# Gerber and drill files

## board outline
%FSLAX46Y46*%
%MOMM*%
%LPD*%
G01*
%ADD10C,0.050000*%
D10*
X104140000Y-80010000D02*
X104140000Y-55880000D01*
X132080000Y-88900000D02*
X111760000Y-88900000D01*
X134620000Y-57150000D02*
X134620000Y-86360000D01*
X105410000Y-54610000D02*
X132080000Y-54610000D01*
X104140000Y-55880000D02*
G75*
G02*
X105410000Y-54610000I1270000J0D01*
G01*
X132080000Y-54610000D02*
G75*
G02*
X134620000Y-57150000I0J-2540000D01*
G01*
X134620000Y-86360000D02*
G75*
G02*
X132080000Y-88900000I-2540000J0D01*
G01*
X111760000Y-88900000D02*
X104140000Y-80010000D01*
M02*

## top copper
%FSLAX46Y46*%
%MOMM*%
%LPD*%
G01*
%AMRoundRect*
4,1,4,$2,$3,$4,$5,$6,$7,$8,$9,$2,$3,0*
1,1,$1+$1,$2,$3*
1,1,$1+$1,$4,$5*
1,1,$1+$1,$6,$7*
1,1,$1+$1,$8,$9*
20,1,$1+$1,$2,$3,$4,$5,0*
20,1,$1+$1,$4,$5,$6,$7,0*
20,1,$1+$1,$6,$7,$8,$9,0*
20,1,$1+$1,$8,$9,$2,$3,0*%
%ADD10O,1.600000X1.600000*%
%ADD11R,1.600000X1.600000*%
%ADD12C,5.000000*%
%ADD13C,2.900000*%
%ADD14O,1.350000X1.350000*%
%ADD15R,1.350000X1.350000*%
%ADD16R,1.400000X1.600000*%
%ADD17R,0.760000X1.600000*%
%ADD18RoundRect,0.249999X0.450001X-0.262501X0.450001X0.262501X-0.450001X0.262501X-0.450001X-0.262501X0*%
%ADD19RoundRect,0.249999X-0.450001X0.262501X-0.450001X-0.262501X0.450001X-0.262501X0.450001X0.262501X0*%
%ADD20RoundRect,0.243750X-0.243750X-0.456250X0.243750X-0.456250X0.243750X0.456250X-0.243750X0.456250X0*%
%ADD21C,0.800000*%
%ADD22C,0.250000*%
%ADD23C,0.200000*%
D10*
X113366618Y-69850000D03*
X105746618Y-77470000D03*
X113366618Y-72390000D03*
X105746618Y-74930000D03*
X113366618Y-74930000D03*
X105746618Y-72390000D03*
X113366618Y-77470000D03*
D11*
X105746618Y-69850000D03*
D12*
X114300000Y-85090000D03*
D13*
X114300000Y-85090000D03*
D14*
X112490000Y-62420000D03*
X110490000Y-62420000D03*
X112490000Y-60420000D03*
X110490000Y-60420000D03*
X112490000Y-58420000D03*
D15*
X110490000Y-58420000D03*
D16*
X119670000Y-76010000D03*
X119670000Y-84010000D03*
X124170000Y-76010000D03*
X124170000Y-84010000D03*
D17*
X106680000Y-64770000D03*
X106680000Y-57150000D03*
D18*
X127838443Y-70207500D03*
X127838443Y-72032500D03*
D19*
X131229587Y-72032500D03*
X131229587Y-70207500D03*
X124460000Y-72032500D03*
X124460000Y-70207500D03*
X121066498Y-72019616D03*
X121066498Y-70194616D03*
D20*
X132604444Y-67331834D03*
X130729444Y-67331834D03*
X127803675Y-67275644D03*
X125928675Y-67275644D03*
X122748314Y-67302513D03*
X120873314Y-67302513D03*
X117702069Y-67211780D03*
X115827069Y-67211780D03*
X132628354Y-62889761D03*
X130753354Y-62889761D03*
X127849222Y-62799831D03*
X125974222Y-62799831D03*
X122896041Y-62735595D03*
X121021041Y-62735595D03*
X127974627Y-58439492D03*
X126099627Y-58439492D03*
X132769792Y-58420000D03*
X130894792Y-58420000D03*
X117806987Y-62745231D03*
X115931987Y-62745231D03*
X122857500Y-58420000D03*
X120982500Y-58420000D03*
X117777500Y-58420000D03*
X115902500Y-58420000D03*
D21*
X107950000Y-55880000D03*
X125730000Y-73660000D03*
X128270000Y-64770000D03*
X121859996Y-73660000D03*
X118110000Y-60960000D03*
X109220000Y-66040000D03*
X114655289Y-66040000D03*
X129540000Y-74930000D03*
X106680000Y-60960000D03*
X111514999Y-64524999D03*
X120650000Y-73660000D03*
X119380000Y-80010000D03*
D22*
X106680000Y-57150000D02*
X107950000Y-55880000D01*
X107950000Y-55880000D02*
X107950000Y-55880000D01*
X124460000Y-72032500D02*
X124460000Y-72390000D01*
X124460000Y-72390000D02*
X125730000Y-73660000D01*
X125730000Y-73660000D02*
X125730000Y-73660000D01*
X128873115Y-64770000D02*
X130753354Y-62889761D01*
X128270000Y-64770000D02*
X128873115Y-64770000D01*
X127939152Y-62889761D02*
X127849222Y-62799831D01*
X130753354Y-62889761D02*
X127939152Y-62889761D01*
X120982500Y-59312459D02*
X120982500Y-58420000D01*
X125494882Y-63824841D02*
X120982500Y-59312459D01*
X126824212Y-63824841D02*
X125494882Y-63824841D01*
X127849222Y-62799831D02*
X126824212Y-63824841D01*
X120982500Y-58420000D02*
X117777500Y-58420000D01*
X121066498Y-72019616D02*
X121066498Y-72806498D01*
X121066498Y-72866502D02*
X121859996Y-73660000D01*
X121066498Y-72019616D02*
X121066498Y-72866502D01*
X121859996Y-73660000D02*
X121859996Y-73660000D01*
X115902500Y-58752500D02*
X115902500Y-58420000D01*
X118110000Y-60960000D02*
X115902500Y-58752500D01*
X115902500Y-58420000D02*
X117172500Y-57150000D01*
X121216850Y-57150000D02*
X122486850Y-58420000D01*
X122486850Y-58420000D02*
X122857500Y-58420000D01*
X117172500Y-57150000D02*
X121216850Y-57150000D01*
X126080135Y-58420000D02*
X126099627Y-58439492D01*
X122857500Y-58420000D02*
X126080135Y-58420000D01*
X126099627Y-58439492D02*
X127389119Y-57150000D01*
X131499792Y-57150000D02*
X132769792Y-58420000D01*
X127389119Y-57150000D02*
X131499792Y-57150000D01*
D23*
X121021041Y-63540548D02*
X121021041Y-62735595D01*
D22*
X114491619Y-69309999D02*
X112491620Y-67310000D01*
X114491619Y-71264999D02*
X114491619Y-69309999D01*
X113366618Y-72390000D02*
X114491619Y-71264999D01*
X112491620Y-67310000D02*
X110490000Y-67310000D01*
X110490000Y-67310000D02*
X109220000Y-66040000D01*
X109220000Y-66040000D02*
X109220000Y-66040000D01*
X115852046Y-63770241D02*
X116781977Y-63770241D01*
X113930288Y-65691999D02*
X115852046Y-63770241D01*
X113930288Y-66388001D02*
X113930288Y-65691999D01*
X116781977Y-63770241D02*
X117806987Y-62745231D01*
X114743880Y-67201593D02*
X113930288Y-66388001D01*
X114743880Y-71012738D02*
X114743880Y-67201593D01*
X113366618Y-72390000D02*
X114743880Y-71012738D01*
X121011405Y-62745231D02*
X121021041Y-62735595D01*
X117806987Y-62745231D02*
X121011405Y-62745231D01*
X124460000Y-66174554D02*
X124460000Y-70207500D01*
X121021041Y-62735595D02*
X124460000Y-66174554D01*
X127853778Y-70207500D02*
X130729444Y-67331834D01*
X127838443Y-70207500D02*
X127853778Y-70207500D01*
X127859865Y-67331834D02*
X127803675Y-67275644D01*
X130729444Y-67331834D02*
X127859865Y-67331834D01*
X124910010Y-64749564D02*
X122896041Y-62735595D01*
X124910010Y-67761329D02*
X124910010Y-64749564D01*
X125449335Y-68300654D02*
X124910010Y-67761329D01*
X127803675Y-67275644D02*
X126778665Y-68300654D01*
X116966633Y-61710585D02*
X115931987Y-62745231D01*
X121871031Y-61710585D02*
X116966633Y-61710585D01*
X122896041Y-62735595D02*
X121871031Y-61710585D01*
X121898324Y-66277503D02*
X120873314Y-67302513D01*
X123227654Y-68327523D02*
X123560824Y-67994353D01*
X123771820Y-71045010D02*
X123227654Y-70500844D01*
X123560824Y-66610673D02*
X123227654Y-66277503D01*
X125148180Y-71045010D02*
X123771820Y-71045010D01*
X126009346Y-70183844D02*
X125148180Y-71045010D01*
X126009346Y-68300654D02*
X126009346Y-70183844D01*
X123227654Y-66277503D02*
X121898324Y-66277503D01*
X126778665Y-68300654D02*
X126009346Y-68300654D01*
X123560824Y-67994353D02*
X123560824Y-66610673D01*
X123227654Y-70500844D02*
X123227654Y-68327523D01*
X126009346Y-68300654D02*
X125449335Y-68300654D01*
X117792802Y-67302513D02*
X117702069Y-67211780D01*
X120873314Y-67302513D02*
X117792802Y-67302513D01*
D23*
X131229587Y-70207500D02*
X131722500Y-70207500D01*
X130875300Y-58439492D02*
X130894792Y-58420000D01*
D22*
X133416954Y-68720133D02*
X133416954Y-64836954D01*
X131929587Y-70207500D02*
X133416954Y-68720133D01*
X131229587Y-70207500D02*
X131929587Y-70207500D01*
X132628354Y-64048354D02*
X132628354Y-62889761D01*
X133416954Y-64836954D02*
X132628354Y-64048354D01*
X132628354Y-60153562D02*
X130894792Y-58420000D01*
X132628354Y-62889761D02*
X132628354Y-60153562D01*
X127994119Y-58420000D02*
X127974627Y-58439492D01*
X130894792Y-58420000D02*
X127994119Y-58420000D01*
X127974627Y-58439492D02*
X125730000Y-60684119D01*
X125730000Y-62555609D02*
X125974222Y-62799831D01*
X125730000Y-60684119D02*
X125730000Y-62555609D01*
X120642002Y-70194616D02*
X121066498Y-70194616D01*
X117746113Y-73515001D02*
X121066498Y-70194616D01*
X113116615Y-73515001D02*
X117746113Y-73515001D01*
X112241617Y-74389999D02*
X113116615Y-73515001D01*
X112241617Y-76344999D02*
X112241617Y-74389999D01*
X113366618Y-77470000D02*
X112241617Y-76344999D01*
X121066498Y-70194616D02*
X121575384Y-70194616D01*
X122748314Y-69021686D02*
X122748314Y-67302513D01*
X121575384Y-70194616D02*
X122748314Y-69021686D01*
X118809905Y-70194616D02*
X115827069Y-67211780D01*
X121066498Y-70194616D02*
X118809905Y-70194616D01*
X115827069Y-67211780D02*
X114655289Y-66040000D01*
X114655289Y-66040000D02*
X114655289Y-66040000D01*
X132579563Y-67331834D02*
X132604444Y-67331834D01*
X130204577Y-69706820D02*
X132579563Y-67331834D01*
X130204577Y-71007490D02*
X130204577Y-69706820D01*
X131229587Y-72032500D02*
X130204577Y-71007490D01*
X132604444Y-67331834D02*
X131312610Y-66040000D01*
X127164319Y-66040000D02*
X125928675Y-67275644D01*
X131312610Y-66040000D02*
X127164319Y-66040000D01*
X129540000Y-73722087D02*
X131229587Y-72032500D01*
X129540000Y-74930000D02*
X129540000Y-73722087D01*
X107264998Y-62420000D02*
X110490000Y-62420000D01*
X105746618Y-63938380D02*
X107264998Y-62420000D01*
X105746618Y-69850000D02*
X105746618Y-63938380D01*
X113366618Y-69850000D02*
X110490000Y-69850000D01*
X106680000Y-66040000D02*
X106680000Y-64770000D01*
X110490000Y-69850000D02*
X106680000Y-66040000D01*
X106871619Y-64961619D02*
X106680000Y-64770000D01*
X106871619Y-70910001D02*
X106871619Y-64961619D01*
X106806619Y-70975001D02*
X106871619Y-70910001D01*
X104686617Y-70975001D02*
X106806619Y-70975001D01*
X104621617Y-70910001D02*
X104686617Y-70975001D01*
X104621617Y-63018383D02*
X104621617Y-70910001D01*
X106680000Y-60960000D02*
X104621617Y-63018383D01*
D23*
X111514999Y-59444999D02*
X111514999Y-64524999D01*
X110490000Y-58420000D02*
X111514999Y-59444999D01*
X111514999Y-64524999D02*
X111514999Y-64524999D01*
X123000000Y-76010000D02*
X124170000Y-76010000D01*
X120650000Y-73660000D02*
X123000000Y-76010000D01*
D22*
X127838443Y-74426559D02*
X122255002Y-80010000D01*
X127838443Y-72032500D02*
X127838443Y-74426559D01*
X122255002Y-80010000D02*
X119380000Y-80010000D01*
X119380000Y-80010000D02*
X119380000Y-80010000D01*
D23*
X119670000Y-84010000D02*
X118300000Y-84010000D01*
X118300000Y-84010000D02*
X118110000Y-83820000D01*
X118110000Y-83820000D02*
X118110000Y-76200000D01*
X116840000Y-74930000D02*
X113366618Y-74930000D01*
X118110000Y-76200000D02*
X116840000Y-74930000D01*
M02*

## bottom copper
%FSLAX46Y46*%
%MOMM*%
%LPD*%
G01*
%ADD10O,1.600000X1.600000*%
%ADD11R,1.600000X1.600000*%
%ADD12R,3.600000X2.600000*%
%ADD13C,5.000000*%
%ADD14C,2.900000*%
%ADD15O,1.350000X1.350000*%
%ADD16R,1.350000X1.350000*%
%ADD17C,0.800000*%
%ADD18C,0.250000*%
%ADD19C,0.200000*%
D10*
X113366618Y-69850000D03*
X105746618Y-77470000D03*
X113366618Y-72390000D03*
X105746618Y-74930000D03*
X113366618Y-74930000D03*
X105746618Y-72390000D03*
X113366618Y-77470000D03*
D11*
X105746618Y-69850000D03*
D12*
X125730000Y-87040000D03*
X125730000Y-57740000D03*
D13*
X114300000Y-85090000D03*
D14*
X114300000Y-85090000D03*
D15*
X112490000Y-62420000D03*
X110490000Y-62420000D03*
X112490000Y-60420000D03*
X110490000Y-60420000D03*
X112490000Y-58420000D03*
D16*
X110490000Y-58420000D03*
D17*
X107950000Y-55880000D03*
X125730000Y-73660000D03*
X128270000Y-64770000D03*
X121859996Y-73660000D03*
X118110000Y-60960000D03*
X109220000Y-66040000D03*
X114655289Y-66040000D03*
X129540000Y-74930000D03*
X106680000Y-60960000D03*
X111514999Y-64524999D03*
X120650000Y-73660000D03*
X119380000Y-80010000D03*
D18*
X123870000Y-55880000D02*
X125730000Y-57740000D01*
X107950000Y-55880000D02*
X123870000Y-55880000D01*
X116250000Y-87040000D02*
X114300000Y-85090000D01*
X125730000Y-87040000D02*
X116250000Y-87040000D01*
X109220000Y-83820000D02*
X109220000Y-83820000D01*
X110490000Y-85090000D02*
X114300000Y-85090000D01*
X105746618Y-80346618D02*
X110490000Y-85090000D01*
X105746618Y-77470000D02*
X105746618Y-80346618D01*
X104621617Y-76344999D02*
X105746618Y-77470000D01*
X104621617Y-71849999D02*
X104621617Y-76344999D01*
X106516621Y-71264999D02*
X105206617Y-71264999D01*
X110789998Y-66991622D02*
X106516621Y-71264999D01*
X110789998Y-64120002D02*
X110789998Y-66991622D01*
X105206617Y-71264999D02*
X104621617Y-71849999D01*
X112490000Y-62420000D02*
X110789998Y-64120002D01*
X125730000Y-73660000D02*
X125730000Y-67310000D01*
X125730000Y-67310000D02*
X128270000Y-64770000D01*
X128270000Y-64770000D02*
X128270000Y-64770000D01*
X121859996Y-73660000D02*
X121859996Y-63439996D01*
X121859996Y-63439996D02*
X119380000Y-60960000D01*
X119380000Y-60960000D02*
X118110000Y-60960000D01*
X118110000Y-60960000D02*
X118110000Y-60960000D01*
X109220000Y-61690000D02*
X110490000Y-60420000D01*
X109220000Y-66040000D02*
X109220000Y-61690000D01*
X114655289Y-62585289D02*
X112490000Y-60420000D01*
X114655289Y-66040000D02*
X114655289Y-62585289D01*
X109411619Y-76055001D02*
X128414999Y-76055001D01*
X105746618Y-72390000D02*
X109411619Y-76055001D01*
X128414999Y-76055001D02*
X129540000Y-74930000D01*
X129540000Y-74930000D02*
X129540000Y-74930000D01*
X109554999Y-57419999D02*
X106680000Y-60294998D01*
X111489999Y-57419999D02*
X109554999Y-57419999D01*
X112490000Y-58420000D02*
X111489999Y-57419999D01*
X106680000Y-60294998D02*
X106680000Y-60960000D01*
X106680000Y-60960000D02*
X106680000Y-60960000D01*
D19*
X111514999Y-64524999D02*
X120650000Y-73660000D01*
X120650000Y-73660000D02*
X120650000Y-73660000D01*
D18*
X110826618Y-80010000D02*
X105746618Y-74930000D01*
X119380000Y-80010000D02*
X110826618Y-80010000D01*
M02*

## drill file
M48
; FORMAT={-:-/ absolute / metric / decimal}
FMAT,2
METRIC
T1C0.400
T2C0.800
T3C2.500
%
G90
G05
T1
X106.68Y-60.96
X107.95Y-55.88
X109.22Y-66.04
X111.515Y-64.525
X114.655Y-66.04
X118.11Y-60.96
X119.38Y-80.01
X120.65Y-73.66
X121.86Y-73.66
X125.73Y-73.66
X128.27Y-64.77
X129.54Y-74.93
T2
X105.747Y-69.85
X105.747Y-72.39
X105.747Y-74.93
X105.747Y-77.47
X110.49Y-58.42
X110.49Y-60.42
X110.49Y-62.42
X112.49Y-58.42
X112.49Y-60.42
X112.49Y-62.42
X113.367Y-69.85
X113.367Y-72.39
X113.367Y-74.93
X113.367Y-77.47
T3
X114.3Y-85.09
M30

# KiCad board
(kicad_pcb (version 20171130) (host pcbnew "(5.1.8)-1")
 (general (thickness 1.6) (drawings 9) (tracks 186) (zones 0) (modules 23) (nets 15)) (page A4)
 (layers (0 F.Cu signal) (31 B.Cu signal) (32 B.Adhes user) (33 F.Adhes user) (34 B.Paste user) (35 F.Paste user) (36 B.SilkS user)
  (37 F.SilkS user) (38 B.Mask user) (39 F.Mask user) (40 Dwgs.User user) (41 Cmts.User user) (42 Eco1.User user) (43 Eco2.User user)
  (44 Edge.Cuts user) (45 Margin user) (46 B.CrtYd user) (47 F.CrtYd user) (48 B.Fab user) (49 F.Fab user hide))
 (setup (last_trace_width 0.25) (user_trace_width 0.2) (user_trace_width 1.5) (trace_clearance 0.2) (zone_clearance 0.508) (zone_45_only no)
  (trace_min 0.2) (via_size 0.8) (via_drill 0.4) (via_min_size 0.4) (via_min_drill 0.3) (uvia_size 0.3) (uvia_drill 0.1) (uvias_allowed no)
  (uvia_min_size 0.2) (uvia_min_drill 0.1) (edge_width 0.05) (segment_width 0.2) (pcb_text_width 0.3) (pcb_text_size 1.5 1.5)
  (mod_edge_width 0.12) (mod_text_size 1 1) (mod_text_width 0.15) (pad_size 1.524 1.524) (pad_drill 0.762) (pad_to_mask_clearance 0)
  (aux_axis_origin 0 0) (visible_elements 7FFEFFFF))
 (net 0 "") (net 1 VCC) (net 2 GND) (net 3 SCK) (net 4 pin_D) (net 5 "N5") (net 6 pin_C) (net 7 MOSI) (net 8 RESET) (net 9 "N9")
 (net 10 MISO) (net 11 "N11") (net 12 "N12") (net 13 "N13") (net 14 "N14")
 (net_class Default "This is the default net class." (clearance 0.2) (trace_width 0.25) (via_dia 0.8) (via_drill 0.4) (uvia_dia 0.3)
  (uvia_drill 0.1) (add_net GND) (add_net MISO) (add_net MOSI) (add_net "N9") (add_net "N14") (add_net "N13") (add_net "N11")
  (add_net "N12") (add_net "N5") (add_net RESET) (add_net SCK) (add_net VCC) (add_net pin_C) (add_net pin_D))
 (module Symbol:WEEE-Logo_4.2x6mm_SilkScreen (layer F.Cu) (at 129.54 81.28 90)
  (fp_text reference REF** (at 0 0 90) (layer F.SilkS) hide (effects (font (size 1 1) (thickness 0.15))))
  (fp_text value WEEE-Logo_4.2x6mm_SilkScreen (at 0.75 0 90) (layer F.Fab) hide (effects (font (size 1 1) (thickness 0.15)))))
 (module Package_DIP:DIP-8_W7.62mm (layer F.Cu) (at 105.746618 69.85)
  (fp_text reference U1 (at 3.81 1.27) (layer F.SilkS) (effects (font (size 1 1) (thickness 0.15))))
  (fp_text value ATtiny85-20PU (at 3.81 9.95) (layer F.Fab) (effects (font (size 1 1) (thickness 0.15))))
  (pad 8 thru_hole oval (at 7.62 0) (size 1.6 1.6) (drill 0.8) (layers *.Cu *.Mask) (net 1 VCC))
  (pad 4 thru_hole oval (at 0 7.62) (size 1.6 1.6) (drill 0.8) (layers *.Cu *.Mask) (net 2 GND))
  (pad 7 thru_hole oval (at 7.62 2.54) (size 1.6 1.6) (drill 0.8) (layers *.Cu *.Mask) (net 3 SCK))
  (pad 3 thru_hole oval (at 0 5.08) (size 1.6 1.6) (drill 0.8) (layers *.Cu *.Mask) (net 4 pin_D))
  (pad 6 thru_hole oval (at 7.62 5.08) (size 1.6 1.6) (drill 0.8) (layers *.Cu *.Mask) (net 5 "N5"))
  (pad 2 thru_hole oval (at 0 2.54) (size 1.6 1.6) (drill 0.8) (layers *.Cu *.Mask) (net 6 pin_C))
  (pad 5 thru_hole oval (at 7.62 7.62) (size 1.6 1.6) (drill 0.8) (layers *.Cu *.Mask) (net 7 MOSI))
  (pad 1 thru_hole rect (at 0 0) (size 1.6 1.6) (drill 0.8) (layers *.Cu *.Mask) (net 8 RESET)))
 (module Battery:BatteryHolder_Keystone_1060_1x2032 (layer B.Cu) (at 125.73 72.39 270)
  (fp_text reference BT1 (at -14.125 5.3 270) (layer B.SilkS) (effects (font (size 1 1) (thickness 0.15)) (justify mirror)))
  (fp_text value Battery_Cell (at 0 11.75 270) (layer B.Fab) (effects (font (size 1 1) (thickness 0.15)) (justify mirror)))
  (pad 2 smd rect (at 14.65 0 90) (size 2.6 3.6) (layers B.Cu B.Paste B.Mask) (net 2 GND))
  (pad 1 smd rect (at -14.65 0 90) (size 2.6 3.6) (layers B.Cu B.Paste B.Mask) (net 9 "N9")))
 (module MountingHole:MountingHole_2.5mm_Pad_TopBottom (layer F.Cu) (at 114.3 85.09)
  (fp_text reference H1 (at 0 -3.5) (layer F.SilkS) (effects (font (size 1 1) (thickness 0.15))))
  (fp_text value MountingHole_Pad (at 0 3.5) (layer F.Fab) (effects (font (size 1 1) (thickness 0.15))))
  (pad 1 connect circle (at 0 0) (size 5 5) (layers B.Cu B.Mask) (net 2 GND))
  (pad 1 connect circle (at 0 0) (size 5 5) (layers F.Cu F.Mask) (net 2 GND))
  (pad 1 thru_hole circle (at 0 0) (size 2.9 2.9) (drill 2.5) (layers *.Cu *.Mask) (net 2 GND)))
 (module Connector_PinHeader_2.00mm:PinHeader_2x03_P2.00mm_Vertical (layer F.Cu) (at 110.49 58.42)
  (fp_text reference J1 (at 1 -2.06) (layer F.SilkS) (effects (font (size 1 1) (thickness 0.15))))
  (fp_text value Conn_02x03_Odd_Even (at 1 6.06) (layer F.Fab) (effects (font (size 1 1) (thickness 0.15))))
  (pad 6 thru_hole oval (at 2 4) (size 1.35 1.35) (drill 0.8) (layers *.Cu *.Mask) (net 2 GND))
  (pad 5 thru_hole oval (at 0 4) (size 1.35 1.35) (drill 0.8) (layers *.Cu *.Mask) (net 8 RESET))
  (pad 4 thru_hole oval (at 2 2) (size 1.35 1.35) (drill 0.8) (layers *.Cu *.Mask) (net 7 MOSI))
  (pad 3 thru_hole oval (at 0 2) (size 1.35 1.35) (drill 0.8) (layers *.Cu *.Mask) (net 3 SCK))
  (pad 2 thru_hole oval (at 2 0) (size 1.35 1.35) (drill 0.8) (layers *.Cu *.Mask) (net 1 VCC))
  (pad 1 thru_hole rect (at 0 0) (size 1.35 1.35) (drill 0.8) (layers *.Cu *.Mask) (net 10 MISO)))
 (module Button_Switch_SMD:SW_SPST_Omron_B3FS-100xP (layer F.Cu) (at 121.92 80.01 90)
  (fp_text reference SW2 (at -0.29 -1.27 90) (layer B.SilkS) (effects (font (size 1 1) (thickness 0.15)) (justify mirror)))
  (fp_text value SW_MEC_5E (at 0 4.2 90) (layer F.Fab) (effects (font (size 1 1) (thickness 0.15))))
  (pad 2 smd rect (at 4 -2.25 270) (size 1.6 1.4) (layers F.Cu F.Paste F.Mask))
  (pad 1 smd rect (at -4 -2.25 270) (size 1.6 1.4) (layers F.Cu F.Paste F.Mask) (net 5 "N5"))
  (pad 4 smd rect (at 4 2.25 270) (size 1.6 1.4) (layers F.Cu F.Paste F.Mask) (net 10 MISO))
  (pad 3 smd rect (at -4 2.25 270) (size 1.6 1.4) (layers F.Cu F.Paste F.Mask)))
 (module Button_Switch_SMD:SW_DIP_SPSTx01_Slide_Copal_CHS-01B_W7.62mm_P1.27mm (layer F.Cu) (at 106.68 60.96 90)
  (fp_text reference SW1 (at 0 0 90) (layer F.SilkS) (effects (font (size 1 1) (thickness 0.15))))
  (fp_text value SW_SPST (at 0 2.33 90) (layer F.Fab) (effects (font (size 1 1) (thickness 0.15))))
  (pad 1 smd rect (at -3.81 0 90) (size 1.6 0.76) (layers F.Cu F.Paste F.Mask) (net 1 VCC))
  (pad 2 smd rect (at 3.81 0 90) (size 1.6 0.76) (layers F.Cu F.Paste F.Mask) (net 9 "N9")))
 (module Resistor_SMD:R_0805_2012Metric (layer F.Cu) (at 127.838443 71.12 90)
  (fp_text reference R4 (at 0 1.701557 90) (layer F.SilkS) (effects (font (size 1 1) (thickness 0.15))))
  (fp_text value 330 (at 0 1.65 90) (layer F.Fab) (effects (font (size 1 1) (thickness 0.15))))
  (pad 2 smd roundrect (at 0.9125 0 90) (size 1.025 1.4) (layers F.Cu F.Paste F.Mask) (roundrect_rratio 0.2439014634146341) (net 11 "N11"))
  (pad 1 smd roundrect (at -0.9125 0 90) (size 1.025 1.4) (layers F.Cu F.Paste F.Mask) (roundrect_rratio 0.2439014634146341) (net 4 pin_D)))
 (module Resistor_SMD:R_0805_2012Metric (layer F.Cu) (at 131.229587 71.12 270)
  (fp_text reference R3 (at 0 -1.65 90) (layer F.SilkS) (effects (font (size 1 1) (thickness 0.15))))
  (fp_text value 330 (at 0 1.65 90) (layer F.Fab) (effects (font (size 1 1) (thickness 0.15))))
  (pad 2 smd roundrect (at 0.9125 0 270) (size 1.025 1.4) (layers F.Cu F.Paste F.Mask) (roundrect_rratio 0.2439014634146341) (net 6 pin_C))
  (pad 1 smd roundrect (at -0.9125 0 270) (size 1.025 1.4) (layers F.Cu F.Paste F.Mask) (roundrect_rratio 0.2439014634146341) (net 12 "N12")))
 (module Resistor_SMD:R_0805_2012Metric (layer F.Cu) (at 124.46 71.12 270)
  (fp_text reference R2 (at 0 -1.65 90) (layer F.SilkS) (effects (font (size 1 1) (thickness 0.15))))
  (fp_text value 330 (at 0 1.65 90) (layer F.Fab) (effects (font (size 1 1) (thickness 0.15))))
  (pad 2 smd roundrect (at 0.9125 0 270) (size 1.025 1.4) (layers F.Cu F.Paste F.Mask) (roundrect_rratio 0.2439014634146341) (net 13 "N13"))
  (pad 1 smd roundrect (at -0.9125 0 270) (size 1.025 1.4) (layers F.Cu F.Paste F.Mask) (roundrect_rratio 0.2439014634146341) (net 3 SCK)))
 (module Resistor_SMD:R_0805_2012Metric (layer F.Cu) (at 121.066498 71.107116 270)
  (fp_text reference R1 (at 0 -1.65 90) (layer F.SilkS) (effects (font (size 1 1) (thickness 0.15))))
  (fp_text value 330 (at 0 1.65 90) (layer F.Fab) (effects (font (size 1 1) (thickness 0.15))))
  (pad 2 smd roundrect (at 0.9125 0 270) (size 1.025 1.4) (layers F.Cu F.Paste F.Mask) (roundrect_rratio 0.2439014634146341) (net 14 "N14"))
  (pad 1 smd roundrect (at -0.9125 0 270) (size 1.025 1.4) (layers F.Cu F.Paste F.Mask) (roundrect_rratio 0.2439014634146341) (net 7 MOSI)))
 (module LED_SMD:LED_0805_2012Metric (layer F.Cu) (at 131.666944 67.331834)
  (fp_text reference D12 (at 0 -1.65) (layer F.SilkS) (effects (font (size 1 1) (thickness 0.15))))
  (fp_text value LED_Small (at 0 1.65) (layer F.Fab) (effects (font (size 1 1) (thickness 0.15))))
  (pad 2 smd roundrect (at 0.9375 0) (size 0.975 1.4) (layers F.Cu F.Paste F.Mask) (roundrect_rratio 0.25) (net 6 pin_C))
  (pad 1 smd roundrect (at -0.9375 0) (size 0.975 1.4) (layers F.Cu F.Paste F.Mask) (roundrect_rratio 0.25) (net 11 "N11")))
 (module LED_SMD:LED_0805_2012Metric (layer F.Cu) (at 126.866175 67.275644)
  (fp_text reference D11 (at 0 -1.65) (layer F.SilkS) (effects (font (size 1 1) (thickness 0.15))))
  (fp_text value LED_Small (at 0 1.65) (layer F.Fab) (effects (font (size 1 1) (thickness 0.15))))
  (pad 2 smd roundrect (at 0.9375 0) (size 0.975 1.4) (layers F.Cu F.Paste F.Mask) (roundrect_rratio 0.25) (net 11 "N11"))
  (pad 1 smd roundrect (at -0.9375 0) (size 0.975 1.4) (layers F.Cu F.Paste F.Mask) (roundrect_rratio 0.25) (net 6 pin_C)))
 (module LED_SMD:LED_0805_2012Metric (layer F.Cu) (at 121.810814 67.302513)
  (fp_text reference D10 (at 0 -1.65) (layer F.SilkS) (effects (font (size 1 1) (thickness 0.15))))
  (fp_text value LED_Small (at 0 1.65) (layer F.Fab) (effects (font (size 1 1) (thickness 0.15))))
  (pad 2 smd roundrect (at 0.9375 0) (size 0.975 1.4) (layers F.Cu F.Paste F.Mask) (roundrect_rratio 0.25) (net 7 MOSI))
  (pad 1 smd roundrect (at -0.9375 0) (size 0.975 1.4) (layers F.Cu F.Paste F.Mask) (roundrect_rratio 0.25) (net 11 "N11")))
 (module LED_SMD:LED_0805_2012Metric (layer F.Cu) (at 116.764569 67.21178)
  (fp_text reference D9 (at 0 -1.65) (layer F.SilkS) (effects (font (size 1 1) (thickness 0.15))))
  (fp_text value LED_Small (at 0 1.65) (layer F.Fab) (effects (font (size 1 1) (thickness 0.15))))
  (pad 2 smd roundrect (at 0.9375 0) (size 0.975 1.4) (layers F.Cu F.Paste F.Mask) (roundrect_rratio 0.25) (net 11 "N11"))
  (pad 1 smd roundrect (at -0.9375 0) (size 0.975 1.4) (layers F.Cu F.Paste F.Mask) (roundrect_rratio 0.25) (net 7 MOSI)))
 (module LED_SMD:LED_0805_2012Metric (layer F.Cu) (at 131.690854 62.889761)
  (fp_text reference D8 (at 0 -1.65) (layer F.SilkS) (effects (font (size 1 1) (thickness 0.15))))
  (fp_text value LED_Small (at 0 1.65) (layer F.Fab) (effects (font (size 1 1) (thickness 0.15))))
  (pad 2 smd roundrect (at 0.9375 0) (size 0.975 1.4) (layers F.Cu F.Paste F.Mask) (roundrect_rratio 0.25) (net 12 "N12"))
  (pad 1 smd roundrect (at -0.9375 0) (size 0.975 1.4) (layers F.Cu F.Paste F.Mask) (roundrect_rratio 0.25) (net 13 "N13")))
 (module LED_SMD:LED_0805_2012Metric (layer F.Cu) (at 126.911722 62.799831)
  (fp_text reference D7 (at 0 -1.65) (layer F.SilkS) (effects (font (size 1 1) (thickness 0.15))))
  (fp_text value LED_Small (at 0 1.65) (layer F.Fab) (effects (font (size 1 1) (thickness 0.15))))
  (pad 2 smd roundrect (at 0.9375 0) (size 0.975 1.4) (layers F.Cu F.Paste F.Mask) (roundrect_rratio 0.25) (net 13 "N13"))
  (pad 1 smd roundrect (at -0.9375 0) (size 0.975 1.4) (layers F.Cu F.Paste F.Mask) (roundrect_rratio 0.25) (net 12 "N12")))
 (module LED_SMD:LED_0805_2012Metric (layer F.Cu) (at 121.958541 62.735595)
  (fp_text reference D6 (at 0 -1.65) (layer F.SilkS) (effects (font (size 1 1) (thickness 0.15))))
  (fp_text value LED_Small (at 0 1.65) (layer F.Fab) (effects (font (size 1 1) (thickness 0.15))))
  (pad 2 smd roundrect (at 0.9375 0) (size 0.975 1.4) (layers F.Cu F.Paste F.Mask) (roundrect_rratio 0.25) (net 11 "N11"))
  (pad 1 smd roundrect (at -0.9375 0) (size 0.975 1.4) (layers F.Cu F.Paste F.Mask) (roundrect_rratio 0.25) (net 3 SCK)))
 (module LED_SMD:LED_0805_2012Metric (layer F.Cu) (at 127.037127 58.439492)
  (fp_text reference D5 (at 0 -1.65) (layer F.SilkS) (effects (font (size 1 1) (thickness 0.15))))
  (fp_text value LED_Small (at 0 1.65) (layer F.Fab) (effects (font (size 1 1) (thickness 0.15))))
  (pad 2 smd roundrect (at 0.9375 0) (size 0.975 1.4) (layers F.Cu F.Paste F.Mask) (roundrect_rratio 0.25) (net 12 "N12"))
  (pad 1 smd roundrect (at -0.9375 0) (size 0.975 1.4) (layers F.Cu F.Paste F.Mask) (roundrect_rratio 0.25) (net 14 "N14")))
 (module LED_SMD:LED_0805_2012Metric (layer F.Cu) (at 131.832292 58.42)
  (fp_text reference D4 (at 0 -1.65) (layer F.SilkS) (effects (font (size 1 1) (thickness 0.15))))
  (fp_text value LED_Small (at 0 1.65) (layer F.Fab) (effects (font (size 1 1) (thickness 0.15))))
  (pad 2 smd roundrect (at 0.9375 0) (size 0.975 1.4) (layers F.Cu F.Paste F.Mask) (roundrect_rratio 0.25) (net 14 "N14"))
  (pad 1 smd roundrect (at -0.9375 0) (size 0.975 1.4) (layers F.Cu F.Paste F.Mask) (roundrect_rratio 0.25) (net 12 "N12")))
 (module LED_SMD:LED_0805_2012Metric (layer F.Cu) (at 116.869487 62.745231)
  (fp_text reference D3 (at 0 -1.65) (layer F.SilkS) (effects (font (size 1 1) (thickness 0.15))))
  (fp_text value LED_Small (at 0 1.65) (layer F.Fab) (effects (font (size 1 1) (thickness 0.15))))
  (pad 2 smd roundrect (at 0.9375 0) (size 0.975 1.4) (layers F.Cu F.Paste F.Mask) (roundrect_rratio 0.25) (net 3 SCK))
  (pad 1 smd roundrect (at -0.9375 0) (size 0.975 1.4) (layers F.Cu F.Paste F.Mask) (roundrect_rratio 0.25) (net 11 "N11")))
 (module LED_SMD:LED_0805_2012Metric (layer F.Cu) (at 121.92 58.42)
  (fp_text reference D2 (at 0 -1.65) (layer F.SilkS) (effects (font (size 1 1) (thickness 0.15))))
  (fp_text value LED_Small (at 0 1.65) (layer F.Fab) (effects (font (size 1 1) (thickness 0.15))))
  (pad 2 smd roundrect (at 0.9375 0) (size 0.975 1.4) (layers F.Cu F.Paste F.Mask) (roundrect_rratio 0.25) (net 14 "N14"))
  (pad 1 smd roundrect (at -0.9375 0) (size 0.975 1.4) (layers F.Cu F.Paste F.Mask) (roundrect_rratio 0.25) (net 13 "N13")))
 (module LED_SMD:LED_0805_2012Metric (layer F.Cu) (at 116.84 58.42)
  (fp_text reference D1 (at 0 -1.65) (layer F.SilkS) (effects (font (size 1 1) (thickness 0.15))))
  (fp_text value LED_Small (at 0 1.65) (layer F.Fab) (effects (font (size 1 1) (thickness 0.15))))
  (pad 2 smd roundrect (at 0.9375 0) (size 0.975 1.4) (layers F.Cu F.Paste F.Mask) (roundrect_rratio 0.25) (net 13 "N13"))
  (pad 1 smd roundrect (at -0.9375 0) (size 0.975 1.4) (layers F.Cu F.Paste F.Mask) (roundrect_rratio 0.25) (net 14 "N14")))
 (gr_line (start 104.14 80.01) (end 104.14 55.88) (layer Edge.Cuts) (width 0.05))
 (gr_line (start 132.08 88.9) (end 111.76 88.9) (layer Edge.Cuts) (width 0.05))
 (gr_line (start 134.62 57.15) (end 134.62 86.36) (layer Edge.Cuts) (width 0.05))
 (gr_line (start 105.41 54.61) (end 132.08 54.61) (layer Edge.Cuts) (width 0.05))
 (gr_arc (start 105.41 55.88) (end 105.41 54.61) (angle -90) (layer Edge.Cuts) (width 0.05))
 (gr_arc (start 132.08 57.15) (end 134.62 57.15) (angle -90) (layer Edge.Cuts) (width 0.05))
 (gr_arc (start 132.08 86.36) (end 132.08 88.9) (angle -90) (layer Edge.Cuts) (width 0.05))
 (gr_line (start 111.76 88.9) (end 104.14 80.01) (layer Edge.Cuts) (width 0.05))
 (segment (start 106.68 57.15) (end 107.95 55.88) (width 0.25) (layer F.Cu) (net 9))
 (segment (start 107.95 55.88) (end 107.95 55.88) (width 0.25) (layer F.Cu) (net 9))
 (via (at 107.95 55.88) (size 0.8) (drill 0.4) (layers F.Cu B.Cu) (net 9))
 (segment (start 123.87 55.88) (end 125.73 57.74) (width 0.25) (layer B.Cu) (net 9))
 (segment (start 107.95 55.88) (end 123.87 55.88) (width 0.25) (layer B.Cu) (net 9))
 (segment (start 116.25 87.04) (end 114.3 85.09) (width 0.25) (layer B.Cu) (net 2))
 (segment (start 125.73 87.04) (end 116.25 87.04) (width 0.25) (layer B.Cu) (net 2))
 (segment (start 109.22 83.82) (end 109.22 83.82) (width 0.25) (layer B.Cu) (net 2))
 (segment (start 110.49 85.09) (end 114.3 85.09) (width 0.25) (layer B.Cu) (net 2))
 (segment (start 105.746618 80.346618) (end 110.49 85.09) (width 0.25) (layer B.Cu) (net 2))
 (segment (start 105.746618 77.47) (end 105.746618 80.346618) (width 0.25) (layer B.Cu) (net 2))
 (segment (start 104.621617 76.344999) (end 105.746618 77.47) (width 0.25) (layer B.Cu) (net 2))
 (segment (start 104.621617 71.849999) (end 104.621617 76.344999) (width 0.25) (layer B.Cu) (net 2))
 (segment (start 106.516621 71.264999) (end 105.206617 71.264999) (width 0.25) (layer B.Cu) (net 2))
 (segment (start 110.789998 66.991622) (end 106.516621 71.264999) (width 0.25) (layer B.Cu) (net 2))
 (segment (start 110.789998 64.120002) (end 110.789998 66.991622) (width 0.25) (layer B.Cu) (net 2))
 (segment (start 105.206617 71.264999) (end 104.621617 71.849999) (width 0.25) (layer B.Cu) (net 2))
 (segment (start 112.49 62.42) (end 110.789998 64.120002) (width 0.25) (layer B.Cu) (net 2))
 (segment (start 124.46 72.0325) (end 124.46 72.39) (width 0.25) (layer F.Cu) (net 13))
 (segment (start 124.46 72.39) (end 125.73 73.66) (width 0.25) (layer F.Cu) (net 13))
 (segment (start 125.73 73.66) (end 125.73 73.66) (width 0.25) (layer F.Cu) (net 13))
 (via (at 125.73 73.66) (size 0.8) (drill 0.4) (layers F.Cu B.Cu) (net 13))
 (segment (start 125.73 73.66) (end 125.73 67.31) (width 0.25) (layer B.Cu) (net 13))
 (segment (start 125.73 67.31) (end 128.27 64.77) (width 0.25) (layer B.Cu) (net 13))
 (segment (start 128.27 64.77) (end 128.27 64.77) (width 0.25) (layer B.Cu) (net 13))
 (via (at 128.27 64.77) (size 0.8) (drill 0.4) (layers F.Cu B.Cu) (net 13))
 (segment (start 128.873115 64.77) (end 130.753354 62.889761) (width 0.25) (layer F.Cu) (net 13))
 (segment (start 128.27 64.77) (end 128.873115 64.77) (width 0.25) (layer F.Cu) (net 13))
 (segment (start 127.939152 62.889761) (end 127.849222 62.799831) (width 0.25) (layer F.Cu) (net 13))
 (segment (start 130.753354 62.889761) (end 127.939152 62.889761) (width 0.25) (layer F.Cu) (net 13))
 (segment (start 120.9825 59.312459) (end 120.9825 58.42) (width 0.25) (layer F.Cu) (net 13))
 (segment (start 125.494882 63.824841) (end 120.9825 59.312459) (width 0.25) (layer F.Cu) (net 13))
 (segment (start 126.824212 63.824841) (end 125.494882 63.824841) (width 0.25) (layer F.Cu) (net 13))
 (segment (start 127.849222 62.799831) (end 126.824212 63.824841) (width 0.25) (layer F.Cu) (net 13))
 (segment (start 120.9825 58.42) (end 117.7775 58.42) (width 0.25) (layer F.Cu) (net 13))
 (segment (start 121.066498 72.019616) (end 121.066498 72.806498) (width 0.25) (layer F.Cu) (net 14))
 (segment (start 121.066498 72.866502) (end 121.859996 73.66) (width 0.25) (layer F.Cu) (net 14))
 (segment (start 121.066498 72.019616) (end 121.066498 72.866502) (width 0.25) (layer F.Cu) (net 14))
 (segment (start 121.859996 73.66) (end 121.859996 73.66) (width 0.25) (layer F.Cu) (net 14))
 (via (at 121.859996 73.66) (size 0.8) (drill 0.4) (layers F.Cu B.Cu) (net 14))
 (segment (start 121.859996 73.66) (end 121.859996 63.439996) (width 0.25) (layer B.Cu) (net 14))
 (segment (start 121.859996 63.439996) (end 119.38 60.96) (width 0.25) (layer B.Cu) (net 14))
 (segment (start 119.38 60.96) (end 118.11 60.96) (width 0.25) (layer B.Cu) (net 14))
 (segment (start 118.11 60.96) (end 118.11 60.96) (width 0.25) (layer B.Cu) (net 14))
 (via (at 118.11 60.96) (size 0.8) (drill 0.4) (layers F.Cu B.Cu) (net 14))
 (segment (start 115.9025 58.7525) (end 115.9025 58.42) (width 0.25) (layer F.Cu) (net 14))
 (segment (start 118.11 60.96) (end 115.9025 58.7525) (width 0.25) (layer F.Cu) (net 14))
 (segment (start 115.9025 58.42) (end 117.1725 57.15) (width 0.25) (layer F.Cu) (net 14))
 (segment (start 121.21685 57.15) (end 122.48685 58.42) (width 0.25) (layer F.Cu) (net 14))
 (segment (start 122.48685 58.42) (end 122.8575 58.42) (width 0.25) (layer F.Cu) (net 14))
 (segment (start 117.1725 57.15) (end 121.21685 57.15) (width 0.25) (layer F.Cu) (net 14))
 (segment (start 126.080135 58.42) (end 126.099627 58.439492) (width 0.25) (layer F.Cu) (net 14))
 (segment (start 122.8575 58.42) (end 126.080135 58.42) (width 0.25) (layer F.Cu) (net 14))
 (segment (start 126.099627 58.439492) (end 127.389119 57.15) (width 0.25) (layer F.Cu) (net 14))
 (segment (start 131.499792 57.15) (end 132.769792 58.42) (width 0.25) (layer F.Cu) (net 14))
 (segment (start 127.389119 57.15) (end 131.499792 57.15) (width 0.25) (layer F.Cu) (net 14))
 (segment (start 121.021041 63.540548) (end 121.021041 62.735595) (width 0.2) (layer F.Cu) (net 3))
 (segment (start 114.491619 69.309999) (end 112.49162 67.31) (width 0.25) (layer F.Cu) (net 3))
 (segment (start 114.491619 71.264999) (end 114.491619 69.309999) (width 0.25) (layer F.Cu) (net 3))
 (segment (start 113.366618 72.39) (end 114.491619 71.264999) (width 0.25) (layer F.Cu) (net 3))
 (segment (start 112.49162 67.31) (end 110.49 67.31) (width 0.25) (layer F.Cu) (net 3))
 (segment (start 110.49 67.31) (end 109.22 66.04) (width 0.25) (layer F.Cu) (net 3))
 (segment (start 109.22 66.04) (end 109.22 66.04) (width 0.25) (layer F.Cu) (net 3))
 (via (at 109.22 66.04) (size 0.8) (drill 0.4) (layers F.Cu B.Cu) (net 3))
 (segment (start 109.22 61.69) (end 110.49 60.42) (width 0.25) (layer B.Cu) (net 3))
 (segment (start 109.22 66.04) (end 109.22 61.69) (width 0.25) (layer B.Cu) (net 3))
 (segment (start 115.852046 63.770241) (end 116.781977 63.770241) (width 0.25) (layer F.Cu) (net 3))
 (segment (start 113.930288 65.691999) (end 115.852046 63.770241) (width 0.25) (layer F.Cu) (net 3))
 (segment (start 113.930288 66.388001) (end 113.930288 65.691999) (width 0.25) (layer F.Cu) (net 3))
 (segment (start 116.781977 63.770241) (end 117.806987 62.745231) (width 0.25) (layer F.Cu) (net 3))
 (segment (start 114.74388 67.201593) (end 113.930288 66.388001) (width 0.25) (layer F.Cu) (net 3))
 (segment (start 114.74388 71.012738) (end 114.74388 67.201593) (width 0.25) (layer F.Cu) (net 3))
 (segment (start 113.366618 72.39) (end 114.74388 71.012738) (width 0.25) (layer F.Cu) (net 3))
 (segment (start 121.011405 62.745231) (end 121.021041 62.735595) (width 0.25) (layer F.Cu) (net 3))
 (segment (start 117.806987 62.745231) (end 121.011405 62.745231) (width 0.25) (layer F.Cu) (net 3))
 (segment (start 124.46 66.174554) (end 124.46 70.2075) (width 0.25) (layer F.Cu) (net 3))
 (segment (start 121.021041 62.735595) (end 124.46 66.174554) (width 0.25) (layer F.Cu) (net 3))
 (segment (start 127.853778 70.2075) (end 130.729444 67.331834) (width 0.25) (layer F.Cu) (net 11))
 (segment (start 127.838443 70.2075) (end 127.853778 70.2075) (width 0.25) (layer F.Cu) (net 11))
 (segment (start 127.859865 67.331834) (end 127.803675 67.275644) (width 0.25) (layer F.Cu) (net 11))
 (segment (start 130.729444 67.331834) (end 127.859865 67.331834) (width 0.25) (layer F.Cu) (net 11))
 (segment (start 124.91001 64.749564) (end 122.896041 62.735595) (width 0.25) (layer F.Cu) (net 11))
 (segment (start 124.91001 67.761329) (end 124.91001 64.749564) (width 0.25) (layer F.Cu) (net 11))
 (segment (start 125.449335 68.300654) (end 124.91001 67.761329) (width 0.25) (layer F.Cu) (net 11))
 (segment (start 127.803675 67.275644) (end 126.778665 68.300654) (width 0.25) (layer F.Cu) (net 11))
 (segment (start 116.966633 61.710585) (end 115.931987 62.745231) (width 0.25) (layer F.Cu) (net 11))
 (segment (start 121.871031 61.710585) (end 116.966633 61.710585) (width 0.25) (layer F.Cu) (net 11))
 (segment (start 122.896041 62.735595) (end 121.871031 61.710585) (width 0.25) (layer F.Cu) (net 11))
 (segment (start 121.898324 66.277503) (end 120.873314 67.302513) (width 0.25) (layer F.Cu) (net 11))
 (segment (start 123.227654 68.327523) (end 123.560824 67.994353) (width 0.25) (layer F.Cu) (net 11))
 (segment (start 123.77182 71.04501) (end 123.227654 70.500844) (width 0.25) (layer F.Cu) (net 11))
 (segment (start 123.560824 66.610673) (end 123.227654 66.277503) (width 0.25) (layer F.Cu) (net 11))
 (segment (start 125.14818 71.04501) (end 123.77182 71.04501) (width 0.25) (layer F.Cu) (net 11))
 (segment (start 126.009346 70.183844) (end 125.14818 71.04501) (width 0.25) (layer F.Cu) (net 11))
 (segment (start 126.009346 68.300654) (end 126.009346 70.183844) (width 0.25) (layer F.Cu) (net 11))
 (segment (start 123.227654 66.277503) (end 121.898324 66.277503) (width 0.25) (layer F.Cu) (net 11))
 (segment (start 126.778665 68.300654) (end 126.009346 68.300654) (width 0.25) (layer F.Cu) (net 11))
 (segment (start 123.560824 67.994353) (end 123.560824 66.610673) (width 0.25) (layer F.Cu) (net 11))
 (segment (start 123.227654 70.500844) (end 123.227654 68.327523) (width 0.25) (layer F.Cu) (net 11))
 (segment (start 126.009346 68.300654) (end 125.449335 68.300654) (width 0.25) (layer F.Cu) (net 11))
 (segment (start 117.792802 67.302513) (end 117.702069 67.21178) (width 0.25) (layer F.Cu) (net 11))
 (segment (start 120.873314 67.302513) (end 117.792802 67.302513) (width 0.25) (layer F.Cu) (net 11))
 (segment (start 131.229587 70.2075) (end 131.7225 70.2075) (width 0.2) (layer F.Cu) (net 12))
 (segment (start 130.8753 58.439492) (end 130.894792 58.42) (width 0.2) (layer F.Cu) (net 12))
 (segment (start 133.416954 68.720133) (end 133.416954 64.836954) (width 0.25) (layer F.Cu) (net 12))
 (segment (start 131.929587 70.2075) (end 133.416954 68.720133) (width 0.25) (layer F.Cu) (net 12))
 (segment (start 131.229587 70.2075) (end 131.929587 70.2075) (width 0.25) (layer F.Cu) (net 12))
 (segment (start 132.628354 64.048354) (end 132.628354 62.889761) (width 0.25) (layer F.Cu) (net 12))
 (segment (start 133.416954 64.836954) (end 132.628354 64.048354) (width 0.25) (layer F.Cu) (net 12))
 (segment (start 132.628354 60.153562) (end 130.894792 58.42) (width 0.25) (layer F.Cu) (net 12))
 (segment (start 132.628354 62.889761) (end 132.628354 60.153562) (width 0.25) (layer F.Cu) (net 12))
 (segment (start 127.994119 58.42) (end 127.974627 58.439492) (width 0.25) (layer F.Cu) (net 12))
 (segment (start 130.894792 58.42) (end 127.994119 58.42) (width 0.25) (layer F.Cu) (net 12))
 (segment (start 127.974627 58.439492) (end 125.73 60.684119) (width 0.25) (layer F.Cu) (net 12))
 (segment (start 125.73 62.555609) (end 125.974222 62.799831) (width 0.25) (layer F.Cu) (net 12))
 (segment (start 125.73 60.684119) (end 125.73 62.555609) (width 0.25) (layer F.Cu) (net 12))
 (segment (start 120.642002 70.194616) (end 121.066498 70.194616) (width 0.25) (layer F.Cu) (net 7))
 (segment (start 117.746113 73.515001) (end 121.066498 70.194616) (width 0.25) (layer F.Cu) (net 7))
 (segment (start 113.116615 73.515001) (end 117.746113 73.515001) (width 0.25) (layer F.Cu) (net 7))
 (segment (start 112.241617 74.389999) (end 113.116615 73.515001) (width 0.25) (layer F.Cu) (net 7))
 (segment (start 112.241617 76.344999) (end 112.241617 74.389999) (width 0.25) (layer F.Cu) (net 7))
 (segment (start 113.366618 77.47) (end 112.241617 76.344999) (width 0.25) (layer F.Cu) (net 7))
 (segment (start 121.066498 70.194616) (end 121.575384 70.194616) (width 0.25) (layer F.Cu) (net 7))
 (segment (start 122.748314 69.021686) (end 122.748314 67.302513) (width 0.25) (layer F.Cu) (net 7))
 (segment (start 121.575384 70.194616) (end 122.748314 69.021686) (width 0.25) (layer F.Cu) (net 7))
 (segment (start 118.809905 70.194616) (end 115.827069 67.21178) (width 0.25) (layer F.Cu) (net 7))
 (segment (start 121.066498 70.194616) (end 118.809905 70.194616) (width 0.25) (layer F.Cu) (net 7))
 (segment (start 115.827069 67.21178) (end 114.655289 66.04) (width 0.25) (layer F.Cu) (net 7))
 (segment (start 114.655289 66.04) (end 114.655289 66.04) (width 0.25) (layer F.Cu) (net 7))
 (via (at 114.655289 66.04) (size 0.8) (drill 0.4) (layers F.Cu B.Cu) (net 7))
 (segment (start 114.655289 62.585289) (end 112.49 60.42) (width 0.25) (layer B.Cu) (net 7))
 (segment (start 114.655289 66.04) (end 114.655289 62.585289) (width 0.25) (layer B.Cu) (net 7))
 (segment (start 132.579563 67.331834) (end 132.604444 67.331834) (width 0.25) (layer F.Cu) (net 6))
 (segment (start 130.204577 69.70682) (end 132.579563 67.331834) (width 0.25) (layer F.Cu) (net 6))
 (segment (start 130.204577 71.00749) (end 130.204577 69.70682) (width 0.25) (layer F.Cu) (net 6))
 (segment (start 131.229587 72.0325) (end 130.204577 71.00749) (width 0.25) (layer F.Cu) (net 6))
 (segment (start 132.604444 67.331834) (end 131.31261 66.04) (width 0.25) (layer F.Cu) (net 6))
 (segment (start 127.164319 66.04) (end 125.928675 67.275644) (width 0.25) (layer F.Cu) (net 6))
 (segment (start 131.31261 66.04) (end 127.164319 66.04) (width 0.25) (layer F.Cu) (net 6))
 (segment (start 109.411619 76.055001) (end 128.414999 76.055001) (width 0.25) (layer B.Cu) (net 6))
 (segment (start 105.746618 72.39) (end 109.411619 76.055001) (width 0.25) (layer B.Cu) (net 6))
 (segment (start 128.414999 76.055001) (end 129.54 74.93) (width 0.25) (layer B.Cu) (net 6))
 (segment (start 129.54 74.93) (end 129.54 74.93) (width 0.25) (layer B.Cu) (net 6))
 (via (at 129.54 74.93) (size 0.8) (drill 0.4) (layers F.Cu B.Cu) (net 6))
 (segment (start 129.54 73.722087) (end 131.229587 72.0325) (width 0.25) (layer F.Cu) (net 6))
 (segment (start 129.54 74.93) (end 129.54 73.722087) (width 0.25) (layer F.Cu) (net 6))
 (segment (start 107.264998 62.42) (end 110.49 62.42) (width 0.25) (layer F.Cu) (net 8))
 (segment (start 105.746618 63.93838) (end 107.264998 62.42) (width 0.25) (layer F.Cu) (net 8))
 (segment (start 105.746618 69.85) (end 105.746618 63.93838) (width 0.25) (layer F.Cu) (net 8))
 (segment (start 113.366618 69.85) (end 110.49 69.85) (width 0.25) (layer F.Cu) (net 1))
 (segment (start 106.68 66.04) (end 106.68 64.77) (width 0.25) (layer F.Cu) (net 1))
 (segment (start 110.49 69.85) (end 106.68 66.04) (width 0.25) (layer F.Cu) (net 1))
 (segment (start 109.554999 57.419999) (end 106.68 60.294998) (width 0.25) (layer B.Cu) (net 1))
 (segment (start 111.489999 57.419999) (end 109.554999 57.419999) (width 0.25) (layer B.Cu) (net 1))
 (segment (start 112.49 58.42) (end 111.489999 57.419999) (width 0.25) (layer B.Cu) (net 1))
 (segment (start 106.68 60.294998) (end 106.68 60.96) (width 0.25) (layer B.Cu) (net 1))
 (segment (start 106.68 60.96) (end 106.68 60.96) (width 0.25) (layer B.Cu) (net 1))
 (via (at 106.68 60.96) (size 0.8) (drill 0.4) (layers F.Cu B.Cu) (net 1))
 (segment (start 106.871619 64.961619) (end 106.68 64.77) (width 0.25) (layer F.Cu) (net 1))
 (segment (start 106.871619 70.910001) (end 106.871619 64.961619) (width 0.25) (layer F.Cu) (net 1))
 (segment (start 106.806619 70.975001) (end 106.871619 70.910001) (width 0.25) (layer F.Cu) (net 1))
 (segment (start 104.686617 70.975001) (end 106.806619 70.975001) (width 0.25) (layer F.Cu) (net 1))
 (segment (start 104.621617 70.910001) (end 104.686617 70.975001) (width 0.25) (layer F.Cu) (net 1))
 (segment (start 104.621617 63.018383) (end 104.621617 70.910001) (width 0.25) (layer F.Cu) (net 1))
 (segment (start 106.68 60.96) (end 104.621617 63.018383) (width 0.25) (layer F.Cu) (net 1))
 (segment (start 111.514999 59.444999) (end 111.514999 64.524999) (width 0.2) (layer F.Cu) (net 10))
 (segment (start 110.49 58.42) (end 111.514999 59.444999) (width 0.2) (layer F.Cu) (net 10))
 (segment (start 111.514999 64.524999) (end 111.514999 64.524999) (width 0.2) (layer F.Cu) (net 10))
 (via (at 111.514999 64.524999) (size 0.8) (drill 0.4) (layers F.Cu B.Cu) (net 10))
 (segment (start 111.514999 64.524999) (end 120.65 73.66) (width 0.2) (layer B.Cu) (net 10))
 (segment (start 120.65 73.66) (end 120.65 73.66) (width 0.2) (layer B.Cu) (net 10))
 (via (at 120.65 73.66) (size 0.8) (drill 0.4) (layers F.Cu B.Cu) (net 10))
 (segment (start 123 76.01) (end 124.17 76.01) (width 0.2) (layer F.Cu) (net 10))
 (segment (start 120.65 73.66) (end 123 76.01) (width 0.2) (layer F.Cu) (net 10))
 (segment (start 127.838443 74.426559) (end 122.255002 80.01) (width 0.25) (layer F.Cu) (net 4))
 (segment (start 127.838443 72.0325) (end 127.838443 74.426559) (width 0.25) (layer F.Cu) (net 4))
 (segment (start 122.255002 80.01) (end 119.38 80.01) (width 0.25) (layer F.Cu) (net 4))
 (segment (start 119.38 80.01) (end 119.38 80.01) (width 0.25) (layer F.Cu) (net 4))
 (via (at 119.38 80.01) (size 0.8) (drill 0.4) (layers F.Cu B.Cu) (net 4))
 (segment (start 110.826618 80.01) (end 105.746618 74.93) (width 0.25) (layer B.Cu) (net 4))
 (segment (start 119.38 80.01) (end 110.826618 80.01) (width 0.25) (layer B.Cu) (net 4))
 (segment (start 119.67 84.01) (end 118.3 84.01) (width 0.2) (layer F.Cu) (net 5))
 (segment (start 118.3 84.01) (end 118.11 83.82) (width 0.2) (layer F.Cu) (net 5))
 (segment (start 118.11 83.82) (end 118.11 76.2) (width 0.2) (layer F.Cu) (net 5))
 (segment (start 116.84 74.93) (end 113.366618 74.93) (width 0.2) (layer F.Cu) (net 5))
 (segment (start 118.11 76.2) (end 116.84 74.93) (width 0.2) (layer F.Cu) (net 5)))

